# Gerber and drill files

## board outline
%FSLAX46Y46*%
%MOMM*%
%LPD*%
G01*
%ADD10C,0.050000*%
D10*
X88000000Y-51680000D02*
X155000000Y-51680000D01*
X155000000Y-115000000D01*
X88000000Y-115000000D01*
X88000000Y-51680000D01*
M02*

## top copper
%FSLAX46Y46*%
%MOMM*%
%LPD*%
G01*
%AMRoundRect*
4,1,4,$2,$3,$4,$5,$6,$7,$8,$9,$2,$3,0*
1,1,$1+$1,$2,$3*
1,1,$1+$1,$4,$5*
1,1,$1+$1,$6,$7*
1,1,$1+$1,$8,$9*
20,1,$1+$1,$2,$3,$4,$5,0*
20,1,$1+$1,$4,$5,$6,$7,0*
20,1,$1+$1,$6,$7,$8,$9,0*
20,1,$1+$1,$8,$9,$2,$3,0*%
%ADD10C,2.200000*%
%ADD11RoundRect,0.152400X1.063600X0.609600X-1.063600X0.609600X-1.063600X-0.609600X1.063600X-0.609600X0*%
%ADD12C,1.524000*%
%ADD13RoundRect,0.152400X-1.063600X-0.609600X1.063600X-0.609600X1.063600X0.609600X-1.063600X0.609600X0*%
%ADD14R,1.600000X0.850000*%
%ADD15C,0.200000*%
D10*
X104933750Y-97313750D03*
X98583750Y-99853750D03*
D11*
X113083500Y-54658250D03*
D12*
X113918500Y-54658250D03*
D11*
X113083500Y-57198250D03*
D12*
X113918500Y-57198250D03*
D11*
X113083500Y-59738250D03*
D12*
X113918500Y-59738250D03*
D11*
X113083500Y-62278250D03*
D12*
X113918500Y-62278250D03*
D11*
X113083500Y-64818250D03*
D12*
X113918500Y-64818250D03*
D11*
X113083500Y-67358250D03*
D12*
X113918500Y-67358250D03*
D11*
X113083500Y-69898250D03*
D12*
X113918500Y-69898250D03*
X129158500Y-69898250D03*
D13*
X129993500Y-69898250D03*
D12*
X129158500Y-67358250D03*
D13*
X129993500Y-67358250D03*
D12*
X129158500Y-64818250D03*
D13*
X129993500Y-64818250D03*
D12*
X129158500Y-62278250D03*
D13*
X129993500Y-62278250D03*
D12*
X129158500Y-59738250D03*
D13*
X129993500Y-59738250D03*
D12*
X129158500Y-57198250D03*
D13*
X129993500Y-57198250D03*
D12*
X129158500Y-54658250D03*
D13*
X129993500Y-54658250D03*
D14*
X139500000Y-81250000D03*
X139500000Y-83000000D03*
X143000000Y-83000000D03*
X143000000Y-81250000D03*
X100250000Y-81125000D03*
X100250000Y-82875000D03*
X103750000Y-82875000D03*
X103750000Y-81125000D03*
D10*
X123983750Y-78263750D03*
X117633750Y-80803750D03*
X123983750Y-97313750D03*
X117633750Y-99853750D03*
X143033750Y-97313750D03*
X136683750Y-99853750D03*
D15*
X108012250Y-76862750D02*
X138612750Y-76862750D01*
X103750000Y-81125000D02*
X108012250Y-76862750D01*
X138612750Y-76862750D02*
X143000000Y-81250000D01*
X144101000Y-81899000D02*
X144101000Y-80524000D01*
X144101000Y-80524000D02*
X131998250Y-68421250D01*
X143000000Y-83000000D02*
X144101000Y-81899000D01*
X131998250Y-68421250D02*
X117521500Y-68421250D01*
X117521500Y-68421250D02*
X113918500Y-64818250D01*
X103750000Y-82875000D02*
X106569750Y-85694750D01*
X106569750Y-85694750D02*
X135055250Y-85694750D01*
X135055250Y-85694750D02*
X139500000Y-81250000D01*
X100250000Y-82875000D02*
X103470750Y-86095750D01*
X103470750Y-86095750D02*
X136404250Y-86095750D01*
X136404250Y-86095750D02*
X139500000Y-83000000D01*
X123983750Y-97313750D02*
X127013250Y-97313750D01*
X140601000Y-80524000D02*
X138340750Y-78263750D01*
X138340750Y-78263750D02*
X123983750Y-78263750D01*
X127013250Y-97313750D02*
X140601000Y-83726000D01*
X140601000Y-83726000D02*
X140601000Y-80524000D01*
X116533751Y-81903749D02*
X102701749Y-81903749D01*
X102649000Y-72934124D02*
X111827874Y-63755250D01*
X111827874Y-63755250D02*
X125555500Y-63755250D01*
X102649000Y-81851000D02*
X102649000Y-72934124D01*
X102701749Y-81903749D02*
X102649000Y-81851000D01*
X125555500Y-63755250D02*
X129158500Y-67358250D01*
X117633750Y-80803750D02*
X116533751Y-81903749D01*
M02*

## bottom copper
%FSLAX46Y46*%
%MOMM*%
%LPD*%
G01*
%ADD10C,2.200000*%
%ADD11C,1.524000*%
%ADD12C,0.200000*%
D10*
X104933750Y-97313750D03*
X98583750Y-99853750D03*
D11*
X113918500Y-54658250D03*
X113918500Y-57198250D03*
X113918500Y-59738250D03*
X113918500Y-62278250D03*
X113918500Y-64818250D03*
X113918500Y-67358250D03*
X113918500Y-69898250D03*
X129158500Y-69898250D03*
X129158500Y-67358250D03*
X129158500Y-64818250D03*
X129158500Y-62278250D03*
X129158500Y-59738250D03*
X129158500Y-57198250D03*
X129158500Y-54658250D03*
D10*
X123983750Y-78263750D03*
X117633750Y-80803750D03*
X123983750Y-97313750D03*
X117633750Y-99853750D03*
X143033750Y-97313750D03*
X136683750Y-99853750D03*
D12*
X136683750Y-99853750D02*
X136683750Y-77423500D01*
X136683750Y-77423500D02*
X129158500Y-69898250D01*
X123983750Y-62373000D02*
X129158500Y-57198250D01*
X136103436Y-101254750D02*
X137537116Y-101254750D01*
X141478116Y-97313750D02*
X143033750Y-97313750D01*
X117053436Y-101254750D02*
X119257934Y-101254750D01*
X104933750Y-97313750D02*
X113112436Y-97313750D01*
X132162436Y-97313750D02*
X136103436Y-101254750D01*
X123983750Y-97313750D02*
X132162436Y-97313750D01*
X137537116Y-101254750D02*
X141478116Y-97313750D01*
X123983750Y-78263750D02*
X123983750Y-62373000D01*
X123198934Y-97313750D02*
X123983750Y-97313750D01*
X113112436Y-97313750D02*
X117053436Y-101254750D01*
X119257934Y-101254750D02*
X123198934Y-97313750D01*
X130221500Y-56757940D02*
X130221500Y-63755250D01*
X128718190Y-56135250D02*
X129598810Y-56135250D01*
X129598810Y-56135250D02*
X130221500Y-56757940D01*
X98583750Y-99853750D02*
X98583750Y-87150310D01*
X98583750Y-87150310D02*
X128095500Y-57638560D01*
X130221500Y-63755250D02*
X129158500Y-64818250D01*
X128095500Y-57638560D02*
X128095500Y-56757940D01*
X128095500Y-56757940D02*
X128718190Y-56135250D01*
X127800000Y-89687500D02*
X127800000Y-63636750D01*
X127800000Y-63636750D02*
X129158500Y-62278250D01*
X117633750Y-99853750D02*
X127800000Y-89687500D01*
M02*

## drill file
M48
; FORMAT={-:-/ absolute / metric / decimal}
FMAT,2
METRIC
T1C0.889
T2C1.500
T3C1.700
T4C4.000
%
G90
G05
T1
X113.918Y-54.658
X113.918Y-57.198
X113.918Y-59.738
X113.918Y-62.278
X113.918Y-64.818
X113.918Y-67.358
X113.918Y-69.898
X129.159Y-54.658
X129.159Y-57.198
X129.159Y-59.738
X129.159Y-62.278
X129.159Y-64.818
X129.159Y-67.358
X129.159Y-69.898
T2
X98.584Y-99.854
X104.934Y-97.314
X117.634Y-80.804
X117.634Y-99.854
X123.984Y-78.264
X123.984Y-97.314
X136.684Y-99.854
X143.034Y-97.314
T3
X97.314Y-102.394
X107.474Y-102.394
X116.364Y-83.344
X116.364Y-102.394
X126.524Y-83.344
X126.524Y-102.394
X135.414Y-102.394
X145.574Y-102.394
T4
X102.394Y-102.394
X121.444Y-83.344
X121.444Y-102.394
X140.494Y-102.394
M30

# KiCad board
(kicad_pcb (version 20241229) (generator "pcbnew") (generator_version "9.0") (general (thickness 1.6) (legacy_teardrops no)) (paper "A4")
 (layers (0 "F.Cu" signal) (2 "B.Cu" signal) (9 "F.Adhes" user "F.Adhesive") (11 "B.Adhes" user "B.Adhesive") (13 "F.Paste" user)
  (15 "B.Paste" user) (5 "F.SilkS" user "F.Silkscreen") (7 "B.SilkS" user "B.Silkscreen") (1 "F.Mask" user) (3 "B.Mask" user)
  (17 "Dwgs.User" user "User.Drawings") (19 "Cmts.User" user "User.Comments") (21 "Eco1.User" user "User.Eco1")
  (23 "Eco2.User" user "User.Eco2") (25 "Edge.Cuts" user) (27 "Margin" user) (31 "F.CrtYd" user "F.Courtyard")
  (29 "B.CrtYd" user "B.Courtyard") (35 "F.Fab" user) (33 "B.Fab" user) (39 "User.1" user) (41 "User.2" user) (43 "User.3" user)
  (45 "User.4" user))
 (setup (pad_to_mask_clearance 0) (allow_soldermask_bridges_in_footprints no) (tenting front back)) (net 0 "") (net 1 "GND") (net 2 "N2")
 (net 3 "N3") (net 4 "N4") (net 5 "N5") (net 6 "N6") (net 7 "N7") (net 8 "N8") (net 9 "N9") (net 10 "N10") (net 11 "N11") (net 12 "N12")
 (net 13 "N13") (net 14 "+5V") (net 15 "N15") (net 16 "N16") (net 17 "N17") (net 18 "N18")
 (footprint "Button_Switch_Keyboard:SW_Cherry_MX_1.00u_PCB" (layer "F.Cu") (at 104.93375 97.31375)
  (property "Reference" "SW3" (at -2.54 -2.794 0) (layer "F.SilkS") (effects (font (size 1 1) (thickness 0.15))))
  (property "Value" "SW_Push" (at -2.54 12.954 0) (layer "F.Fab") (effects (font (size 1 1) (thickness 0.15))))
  (pad "" np_thru_hole circle (at -7.62 5.08) (size 1.7 1.7) (drill 1.7) (layers "*.Cu" "*.Mask"))
  (pad "" np_thru_hole circle (at -2.54 5.08) (size 4 4) (drill 4) (layers "*.Cu" "*.Mask"))
  (pad "" np_thru_hole circle (at 2.54 5.08) (size 1.7 1.7) (drill 1.7) (layers "*.Cu" "*.Mask"))
  (pad "1" thru_hole circle (at 0 0) (size 2.2 2.2) (drill 1.5) (layers "*.Cu" "*.Mask") (remove_unused_layers no) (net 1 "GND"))
  (pad "2" thru_hole circle (at -6.35 2.54) (size 2.2 2.2) (drill 1.5) (layers "*.Cu" "*.Mask") (remove_unused_layers no) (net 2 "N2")))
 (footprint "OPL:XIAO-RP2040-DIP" (layer "F.Cu") (at 121.5385 62.27825)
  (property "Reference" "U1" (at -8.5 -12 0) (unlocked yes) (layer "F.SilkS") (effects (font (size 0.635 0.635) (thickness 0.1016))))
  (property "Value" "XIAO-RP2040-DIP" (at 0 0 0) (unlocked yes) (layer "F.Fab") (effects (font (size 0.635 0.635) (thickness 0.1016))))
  (pad "1" smd roundrect (at -8.455 -7.62 180) (size 2.432 1.524) (layers "F.Cu" "F.Mask") (roundrect_rratio 0.1) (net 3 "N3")
   (thermal_bridge_angle 45))
  (pad "1" thru_hole circle (at -7.62 -7.62 180) (size 1.524 1.524) (drill 0.889) (layers "*.Cu" "*.Mask") (remove_unused_layers no)
   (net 3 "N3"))
  (pad "2" smd roundrect (at -8.455 -5.08 180) (size 2.432 1.524) (layers "F.Cu" "F.Mask") (roundrect_rratio 0.1) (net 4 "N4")
   (thermal_bridge_angle 45))
  (pad "2" thru_hole circle (at -7.62 -5.08 180) (size 1.524 1.524) (drill 0.889) (layers "*.Cu" "*.Mask") (remove_unused_layers no)
   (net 4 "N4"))
  (pad "3" smd roundrect (at -8.455 -2.54 180) (size 2.432 1.524) (layers "F.Cu" "F.Mask") (roundrect_rratio 0.1) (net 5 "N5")
   (thermal_bridge_angle 45))
  (pad "3" thru_hole circle (at -7.62 -2.54 180) (size 1.524 1.524) (drill 0.889) (layers "*.Cu" "*.Mask") (remove_unused_layers no)
   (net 5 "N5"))
  (pad "4" smd roundrect (at -8.455 0 180) (size 2.432 1.524) (layers "F.Cu" "F.Mask") (roundrect_rratio 0.1) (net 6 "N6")
   (thermal_bridge_angle 45))
  (pad "4" thru_hole circle (at -7.62 0 180) (size 1.524 1.524) (drill 0.889) (layers "*.Cu" "*.Mask") (remove_unused_layers no)
   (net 6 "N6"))
  (pad "5" smd roundrect (at -8.455 2.54 180) (size 2.432 1.524) (layers "F.Cu" "F.Mask") (roundrect_rratio 0.1) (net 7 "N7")
   (thermal_bridge_angle 45))
  (pad "5" thru_hole circle (at -7.62 2.54 180) (size 1.524 1.524) (drill 0.889) (layers "*.Cu" "*.Mask") (remove_unused_layers no)
   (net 7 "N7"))
  (pad "6" smd roundrect (at -8.455 5.08 180) (size 2.432 1.524) (layers "F.Cu" "F.Mask") (roundrect_rratio 0.1) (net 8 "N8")
   (thermal_bridge_angle 45))
  (pad "6" thru_hole circle (at -7.62 5.08 180) (size 1.524 1.524) (drill 0.889) (layers "*.Cu" "*.Mask") (remove_unused_layers no)
   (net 8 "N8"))
  (pad "7" smd roundrect (at -8.455 7.62 180) (size 2.432 1.524) (layers "F.Cu" "F.Mask") (roundrect_rratio 0.1) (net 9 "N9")
   (thermal_bridge_angle 45))
  (pad "7" thru_hole circle (at -7.62 7.62 180) (size 1.524 1.524) (drill 0.889) (layers "*.Cu" "*.Mask") (remove_unused_layers no)
   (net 9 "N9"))
  (pad "8" thru_hole circle (at 7.62 7.62) (size 1.524 1.524) (drill 0.889) (layers "*.Cu" "*.Mask") (remove_unused_layers no)
   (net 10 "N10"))
  (pad "8" smd roundrect (at 8.455 7.62) (size 2.432 1.524) (layers "F.Cu" "F.Mask") (roundrect_rratio 0.1) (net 10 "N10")
   (thermal_bridge_angle 45))
  (pad "9" thru_hole circle (at 7.62 5.08) (size 1.524 1.524) (drill 0.889) (layers "*.Cu" "*.Mask") (remove_unused_layers no)
   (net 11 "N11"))
  (pad "9" smd roundrect (at 8.455 5.08) (size 2.432 1.524) (layers "F.Cu" "F.Mask") (roundrect_rratio 0.1) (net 11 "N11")
   (thermal_bridge_angle 45))
  (pad "10" thru_hole circle (at 7.62 2.54) (size 1.524 1.524) (drill 0.889) (layers "*.Cu" "*.Mask") (remove_unused_layers no) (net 2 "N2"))
  (pad "10" smd roundrect (at 8.455 2.54) (size 2.432 1.524) (layers "F.Cu" "F.Mask") (roundrect_rratio 0.1) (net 2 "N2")
   (thermal_bridge_angle 45))
  (pad "11" thru_hole circle (at 7.62 0) (size 1.524 1.524) (drill 0.889) (layers "*.Cu" "*.Mask") (remove_unused_layers no) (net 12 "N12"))
  (pad "11" smd roundrect (at 8.455 0) (size 2.432 1.524) (layers "F.Cu" "F.Mask") (roundrect_rratio 0.1) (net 12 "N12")
   (thermal_bridge_angle 45))
  (pad "12" thru_hole circle (at 7.62 -2.54) (size 1.524 1.524) (drill 0.889) (layers "*.Cu" "*.Mask") (remove_unused_layers no)
   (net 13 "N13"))
  (pad "12" smd roundrect (at 8.455 -2.54) (size 2.432 1.524) (layers "F.Cu" "F.Mask") (roundrect_rratio 0.1) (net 13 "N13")
   (thermal_bridge_angle 45))
  (pad "13" thru_hole circle (at 7.62 -5.08) (size 1.524 1.524) (drill 0.889) (layers "*.Cu" "*.Mask") (remove_unused_layers no)
   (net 1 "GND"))
  (pad "13" smd roundrect (at 8.455 -5.08) (size 2.432 1.524) (layers "F.Cu" "F.Mask") (roundrect_rratio 0.1) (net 1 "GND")
   (thermal_bridge_angle 45))
  (pad "14" thru_hole circle (at 7.62 -7.62) (size 1.524 1.524) (drill 0.889) (layers "*.Cu" "*.Mask") (remove_unused_layers no)
   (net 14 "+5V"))
  (pad "14" smd roundrect (at 8.455 -7.62) (size 2.432 1.524) (layers "F.Cu" "F.Mask") (roundrect_rratio 0.1) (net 14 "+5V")
   (thermal_bridge_angle 45)))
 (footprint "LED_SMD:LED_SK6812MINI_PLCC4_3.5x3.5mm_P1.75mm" (layer "F.Cu") (at 141.25 82.125)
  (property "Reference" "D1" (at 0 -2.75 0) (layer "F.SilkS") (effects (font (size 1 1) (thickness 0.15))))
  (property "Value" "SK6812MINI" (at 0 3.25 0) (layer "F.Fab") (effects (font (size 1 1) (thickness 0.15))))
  (pad "1" smd rect (at -1.75 -0.875) (size 1.6 0.85) (layers "F.Cu" "F.Mask" "F.Paste") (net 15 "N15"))
  (pad "2" smd rect (at -1.75 0.875) (size 1.6 0.85) (layers "F.Cu" "F.Mask" "F.Paste") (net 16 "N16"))
  (pad "3" smd rect (at 1.75 0.875) (size 1.6 0.85) (layers "F.Cu" "F.Mask" "F.Paste") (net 7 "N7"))
  (pad "4" smd rect (at 1.75 -0.875) (size 1.6 0.85) (layers "F.Cu" "F.Mask" "F.Paste") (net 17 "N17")))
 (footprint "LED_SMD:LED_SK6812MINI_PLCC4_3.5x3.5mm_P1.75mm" (layer "F.Cu") (at 102 82)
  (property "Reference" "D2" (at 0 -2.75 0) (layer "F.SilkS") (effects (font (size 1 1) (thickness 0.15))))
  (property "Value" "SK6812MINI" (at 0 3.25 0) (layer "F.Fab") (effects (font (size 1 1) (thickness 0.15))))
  (pad "1" smd rect (at -1.75 -0.875) (size 1.6 0.85) (layers "F.Cu" "F.Mask" "F.Paste") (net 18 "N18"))
  (pad "2" smd rect (at -1.75 0.875) (size 1.6 0.85) (layers "F.Cu" "F.Mask" "F.Paste") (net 16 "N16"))
  (pad "3" smd rect (at 1.75 0.875) (size 1.6 0.85) (layers "F.Cu" "F.Mask" "F.Paste") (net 15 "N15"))
  (pad "4" smd rect (at 1.75 -0.875) (size 1.6 0.85) (layers "F.Cu" "F.Mask" "F.Paste") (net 17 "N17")))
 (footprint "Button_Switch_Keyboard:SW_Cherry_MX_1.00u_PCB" (layer "F.Cu") (at 123.98375 78.26375)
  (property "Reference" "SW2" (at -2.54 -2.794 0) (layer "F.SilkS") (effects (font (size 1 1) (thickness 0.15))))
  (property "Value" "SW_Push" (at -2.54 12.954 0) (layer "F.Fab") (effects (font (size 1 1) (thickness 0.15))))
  (pad "" np_thru_hole circle (at -7.62 5.08) (size 1.7 1.7) (drill 1.7) (layers "*.Cu" "*.Mask"))
  (pad "" np_thru_hole circle (at -2.54 5.08) (size 4 4) (drill 4) (layers "*.Cu" "*.Mask"))
  (pad "" np_thru_hole circle (at 2.54 5.08) (size 1.7 1.7) (drill 1.7) (layers "*.Cu" "*.Mask"))
  (pad "1" thru_hole circle (at 0 0) (size 2.2 2.2) (drill 1.5) (layers "*.Cu" "*.Mask") (remove_unused_layers no) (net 1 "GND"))
  (pad "2" thru_hole circle (at -6.35 2.54) (size 2.2 2.2) (drill 1.5) (layers "*.Cu" "*.Mask") (remove_unused_layers no) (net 11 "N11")))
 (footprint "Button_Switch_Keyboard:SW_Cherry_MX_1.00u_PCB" (layer "F.Cu") (at 123.98375 97.31375)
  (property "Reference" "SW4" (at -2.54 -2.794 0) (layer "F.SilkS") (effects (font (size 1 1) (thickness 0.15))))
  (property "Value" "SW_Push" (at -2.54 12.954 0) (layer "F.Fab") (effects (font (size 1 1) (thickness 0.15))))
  (pad "" np_thru_hole circle (at -7.62 5.08) (size 1.7 1.7) (drill 1.7) (layers "*.Cu" "*.Mask"))
  (pad "" np_thru_hole circle (at -2.54 5.08) (size 4 4) (drill 4) (layers "*.Cu" "*.Mask"))
  (pad "" np_thru_hole circle (at 2.54 5.08) (size 1.7 1.7) (drill 1.7) (layers "*.Cu" "*.Mask"))
  (pad "1" thru_hole circle (at 0 0) (size 2.2 2.2) (drill 1.5) (layers "*.Cu" "*.Mask") (remove_unused_layers no) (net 1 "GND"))
  (pad "2" thru_hole circle (at -6.35 2.54) (size 2.2 2.2) (drill 1.5) (layers "*.Cu" "*.Mask") (remove_unused_layers no) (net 12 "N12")))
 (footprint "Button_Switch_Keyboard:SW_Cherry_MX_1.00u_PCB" (layer "F.Cu") (at 143.03375 97.31375)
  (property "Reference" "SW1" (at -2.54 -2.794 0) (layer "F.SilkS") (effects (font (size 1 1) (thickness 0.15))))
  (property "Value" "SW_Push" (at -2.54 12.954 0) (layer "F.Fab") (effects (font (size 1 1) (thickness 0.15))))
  (pad "" np_thru_hole circle (at -7.62 5.08) (size 1.7 1.7) (drill 1.7) (layers "*.Cu" "*.Mask"))
  (pad "" np_thru_hole circle (at -2.54 5.08) (size 4 4) (drill 4) (layers "*.Cu" "*.Mask"))
  (pad "" np_thru_hole circle (at 2.54 5.08) (size 1.7 1.7) (drill 1.7) (layers "*.Cu" "*.Mask"))
  (pad "1" thru_hole circle (at 0 0) (size 2.2 2.2) (drill 1.5) (layers "*.Cu" "*.Mask") (remove_unused_layers no) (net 1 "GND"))
  (pad "2" thru_hole circle (at -6.35 2.54) (size 2.2 2.2) (drill 1.5) (layers "*.Cu" "*.Mask") (remove_unused_layers no) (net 10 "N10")))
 (gr_rect (start 88 51.68) (end 155 115) (stroke (width 0.05) (type default)) (fill no) (layer "Edge.Cuts"))
 (segment (start 108.01225 76.86275) (end 138.61275 76.86275) (width 0.2) (layer "F.Cu") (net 17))
 (segment (start 103.75 81.125) (end 108.01225 76.86275) (width 0.2) (layer "F.Cu") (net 17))
 (segment (start 138.61275 76.86275) (end 143 81.25) (width 0.2) (layer "F.Cu") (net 17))
 (segment (start 144.101 81.899) (end 144.101 80.524) (width 0.2) (layer "F.Cu") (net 7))
 (segment (start 144.101 80.524) (end 131.99825 68.42125) (width 0.2) (layer "F.Cu") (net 7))
 (segment (start 143 83) (end 144.101 81.899) (width 0.2) (layer "F.Cu") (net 7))
 (segment (start 131.99825 68.42125) (end 117.5215 68.42125) (width 0.2) (layer "F.Cu") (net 7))
 (segment (start 117.5215 68.42125) (end 113.9185 64.81825) (width 0.2) (layer "F.Cu") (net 7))
 (segment (start 103.75 82.875) (end 106.56975 85.69475) (width 0.2) (layer "F.Cu") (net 15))
 (segment (start 106.56975 85.69475) (end 135.05525 85.69475) (width 0.2) (layer "F.Cu") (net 15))
 (segment (start 135.05525 85.69475) (end 139.5 81.25) (width 0.2) (layer "F.Cu") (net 15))
 (segment (start 100.25 82.875) (end 103.47075 86.09575) (width 0.2) (layer "F.Cu") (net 16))
 (segment (start 103.47075 86.09575) (end 136.40425 86.09575) (width 0.2) (layer "F.Cu") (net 16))
 (segment (start 136.40425 86.09575) (end 139.5 83) (width 0.2) (layer "F.Cu") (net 16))
 (segment (start 136.68375 99.85375) (end 136.68375 77.4235) (width 0.2) (layer "B.Cu") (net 10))
 (segment (start 136.68375 77.4235) (end 129.1585 69.89825) (width 0.2) (layer "B.Cu") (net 10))
 (segment (start 123.98375 97.31375) (end 127.01325 97.31375) (width 0.2) (layer "F.Cu") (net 1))
 (segment (start 140.601 80.524) (end 138.34075 78.26375) (width 0.2) (layer "F.Cu") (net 1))
 (segment (start 138.34075 78.26375) (end 123.98375 78.26375) (width 0.2) (layer "F.Cu") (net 1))
 (segment (start 127.01325 97.31375) (end 140.601 83.726) (width 0.2) (layer "F.Cu") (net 1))
 (segment (start 140.601 83.726) (end 140.601 80.524) (width 0.2) (layer "F.Cu") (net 1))
 (segment (start 123.98375 62.373) (end 129.1585 57.19825) (width 0.2) (layer "B.Cu") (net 1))
 (segment (start 136.103436 101.25475) (end 137.537116 101.25475) (width 0.2) (layer "B.Cu") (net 1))
 (segment (start 141.478116 97.31375) (end 143.03375 97.31375) (width 0.2) (layer "B.Cu") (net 1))
 (segment (start 117.053436 101.25475) (end 119.257934 101.25475) (width 0.2) (layer "B.Cu") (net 1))
 (segment (start 104.93375 97.31375) (end 113.112436 97.31375) (width 0.2) (layer "B.Cu") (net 1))
 (segment (start 132.162436 97.31375) (end 136.103436 101.25475) (width 0.2) (layer "B.Cu") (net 1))
 (segment (start 123.98375 97.31375) (end 132.162436 97.31375) (width 0.2) (layer "B.Cu") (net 1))
 (segment (start 137.537116 101.25475) (end 141.478116 97.31375) (width 0.2) (layer "B.Cu") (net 1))
 (segment (start 123.98375 78.26375) (end 123.98375 62.373) (width 0.2) (layer "B.Cu") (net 1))
 (segment (start 123.198934 97.31375) (end 123.98375 97.31375) (width 0.2) (layer "B.Cu") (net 1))
 (segment (start 113.112436 97.31375) (end 117.053436 101.25475) (width 0.2) (layer "B.Cu") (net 1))
 (segment (start 119.257934 101.25475) (end 123.198934 97.31375) (width 0.2) (layer "B.Cu") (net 1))
 (segment (start 116.533751 81.903749) (end 102.701749 81.903749) (width 0.2) (layer "F.Cu") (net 11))
 (segment (start 102.649 72.934124) (end 111.827874 63.75525) (width 0.2) (layer "F.Cu") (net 11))
 (segment (start 111.827874 63.75525) (end 125.5555 63.75525) (width 0.2) (layer "F.Cu") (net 11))
 (segment (start 102.649 81.851) (end 102.649 72.934124) (width 0.2) (layer "F.Cu") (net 11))
 (segment (start 102.701749 81.903749) (end 102.649 81.851) (width 0.2) (layer "F.Cu") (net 11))
 (segment (start 125.5555 63.75525) (end 129.1585 67.35825) (width 0.2) (layer "F.Cu") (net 11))
 (segment (start 117.63375 80.80375) (end 116.533751 81.903749) (width 0.2) (layer "F.Cu") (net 11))
 (segment (start 130.2215 56.75794) (end 130.2215 63.75525) (width 0.2) (layer "B.Cu") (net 2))
 (segment (start 128.71819 56.13525) (end 129.59881 56.13525) (width 0.2) (layer "B.Cu") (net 2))
 (segment (start 129.59881 56.13525) (end 130.2215 56.75794) (width 0.2) (layer "B.Cu") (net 2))
 (segment (start 98.58375 99.85375) (end 98.58375 87.15031) (width 0.2) (layer "B.Cu") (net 2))
 (segment (start 98.58375 87.15031) (end 128.0955 57.63856) (width 0.2) (layer "B.Cu") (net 2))
 (segment (start 130.2215 63.75525) (end 129.1585 64.81825) (width 0.2) (layer "B.Cu") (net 2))
 (segment (start 128.0955 57.63856) (end 128.0955 56.75794) (width 0.2) (layer "B.Cu") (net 2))
 (segment (start 128.0955 56.75794) (end 128.71819 56.13525) (width 0.2) (layer "B.Cu") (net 2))
 (segment (start 127.8 89.6875) (end 127.8 63.63675) (width 0.2) (layer "B.Cu") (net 12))
 (segment (start 127.8 63.63675) (end 129.1585 62.27825) (width 0.2) (layer "B.Cu") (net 12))
 (segment (start 117.63375 99.85375) (end 127.8 89.6875) (width 0.2) (layer "B.Cu") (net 12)))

